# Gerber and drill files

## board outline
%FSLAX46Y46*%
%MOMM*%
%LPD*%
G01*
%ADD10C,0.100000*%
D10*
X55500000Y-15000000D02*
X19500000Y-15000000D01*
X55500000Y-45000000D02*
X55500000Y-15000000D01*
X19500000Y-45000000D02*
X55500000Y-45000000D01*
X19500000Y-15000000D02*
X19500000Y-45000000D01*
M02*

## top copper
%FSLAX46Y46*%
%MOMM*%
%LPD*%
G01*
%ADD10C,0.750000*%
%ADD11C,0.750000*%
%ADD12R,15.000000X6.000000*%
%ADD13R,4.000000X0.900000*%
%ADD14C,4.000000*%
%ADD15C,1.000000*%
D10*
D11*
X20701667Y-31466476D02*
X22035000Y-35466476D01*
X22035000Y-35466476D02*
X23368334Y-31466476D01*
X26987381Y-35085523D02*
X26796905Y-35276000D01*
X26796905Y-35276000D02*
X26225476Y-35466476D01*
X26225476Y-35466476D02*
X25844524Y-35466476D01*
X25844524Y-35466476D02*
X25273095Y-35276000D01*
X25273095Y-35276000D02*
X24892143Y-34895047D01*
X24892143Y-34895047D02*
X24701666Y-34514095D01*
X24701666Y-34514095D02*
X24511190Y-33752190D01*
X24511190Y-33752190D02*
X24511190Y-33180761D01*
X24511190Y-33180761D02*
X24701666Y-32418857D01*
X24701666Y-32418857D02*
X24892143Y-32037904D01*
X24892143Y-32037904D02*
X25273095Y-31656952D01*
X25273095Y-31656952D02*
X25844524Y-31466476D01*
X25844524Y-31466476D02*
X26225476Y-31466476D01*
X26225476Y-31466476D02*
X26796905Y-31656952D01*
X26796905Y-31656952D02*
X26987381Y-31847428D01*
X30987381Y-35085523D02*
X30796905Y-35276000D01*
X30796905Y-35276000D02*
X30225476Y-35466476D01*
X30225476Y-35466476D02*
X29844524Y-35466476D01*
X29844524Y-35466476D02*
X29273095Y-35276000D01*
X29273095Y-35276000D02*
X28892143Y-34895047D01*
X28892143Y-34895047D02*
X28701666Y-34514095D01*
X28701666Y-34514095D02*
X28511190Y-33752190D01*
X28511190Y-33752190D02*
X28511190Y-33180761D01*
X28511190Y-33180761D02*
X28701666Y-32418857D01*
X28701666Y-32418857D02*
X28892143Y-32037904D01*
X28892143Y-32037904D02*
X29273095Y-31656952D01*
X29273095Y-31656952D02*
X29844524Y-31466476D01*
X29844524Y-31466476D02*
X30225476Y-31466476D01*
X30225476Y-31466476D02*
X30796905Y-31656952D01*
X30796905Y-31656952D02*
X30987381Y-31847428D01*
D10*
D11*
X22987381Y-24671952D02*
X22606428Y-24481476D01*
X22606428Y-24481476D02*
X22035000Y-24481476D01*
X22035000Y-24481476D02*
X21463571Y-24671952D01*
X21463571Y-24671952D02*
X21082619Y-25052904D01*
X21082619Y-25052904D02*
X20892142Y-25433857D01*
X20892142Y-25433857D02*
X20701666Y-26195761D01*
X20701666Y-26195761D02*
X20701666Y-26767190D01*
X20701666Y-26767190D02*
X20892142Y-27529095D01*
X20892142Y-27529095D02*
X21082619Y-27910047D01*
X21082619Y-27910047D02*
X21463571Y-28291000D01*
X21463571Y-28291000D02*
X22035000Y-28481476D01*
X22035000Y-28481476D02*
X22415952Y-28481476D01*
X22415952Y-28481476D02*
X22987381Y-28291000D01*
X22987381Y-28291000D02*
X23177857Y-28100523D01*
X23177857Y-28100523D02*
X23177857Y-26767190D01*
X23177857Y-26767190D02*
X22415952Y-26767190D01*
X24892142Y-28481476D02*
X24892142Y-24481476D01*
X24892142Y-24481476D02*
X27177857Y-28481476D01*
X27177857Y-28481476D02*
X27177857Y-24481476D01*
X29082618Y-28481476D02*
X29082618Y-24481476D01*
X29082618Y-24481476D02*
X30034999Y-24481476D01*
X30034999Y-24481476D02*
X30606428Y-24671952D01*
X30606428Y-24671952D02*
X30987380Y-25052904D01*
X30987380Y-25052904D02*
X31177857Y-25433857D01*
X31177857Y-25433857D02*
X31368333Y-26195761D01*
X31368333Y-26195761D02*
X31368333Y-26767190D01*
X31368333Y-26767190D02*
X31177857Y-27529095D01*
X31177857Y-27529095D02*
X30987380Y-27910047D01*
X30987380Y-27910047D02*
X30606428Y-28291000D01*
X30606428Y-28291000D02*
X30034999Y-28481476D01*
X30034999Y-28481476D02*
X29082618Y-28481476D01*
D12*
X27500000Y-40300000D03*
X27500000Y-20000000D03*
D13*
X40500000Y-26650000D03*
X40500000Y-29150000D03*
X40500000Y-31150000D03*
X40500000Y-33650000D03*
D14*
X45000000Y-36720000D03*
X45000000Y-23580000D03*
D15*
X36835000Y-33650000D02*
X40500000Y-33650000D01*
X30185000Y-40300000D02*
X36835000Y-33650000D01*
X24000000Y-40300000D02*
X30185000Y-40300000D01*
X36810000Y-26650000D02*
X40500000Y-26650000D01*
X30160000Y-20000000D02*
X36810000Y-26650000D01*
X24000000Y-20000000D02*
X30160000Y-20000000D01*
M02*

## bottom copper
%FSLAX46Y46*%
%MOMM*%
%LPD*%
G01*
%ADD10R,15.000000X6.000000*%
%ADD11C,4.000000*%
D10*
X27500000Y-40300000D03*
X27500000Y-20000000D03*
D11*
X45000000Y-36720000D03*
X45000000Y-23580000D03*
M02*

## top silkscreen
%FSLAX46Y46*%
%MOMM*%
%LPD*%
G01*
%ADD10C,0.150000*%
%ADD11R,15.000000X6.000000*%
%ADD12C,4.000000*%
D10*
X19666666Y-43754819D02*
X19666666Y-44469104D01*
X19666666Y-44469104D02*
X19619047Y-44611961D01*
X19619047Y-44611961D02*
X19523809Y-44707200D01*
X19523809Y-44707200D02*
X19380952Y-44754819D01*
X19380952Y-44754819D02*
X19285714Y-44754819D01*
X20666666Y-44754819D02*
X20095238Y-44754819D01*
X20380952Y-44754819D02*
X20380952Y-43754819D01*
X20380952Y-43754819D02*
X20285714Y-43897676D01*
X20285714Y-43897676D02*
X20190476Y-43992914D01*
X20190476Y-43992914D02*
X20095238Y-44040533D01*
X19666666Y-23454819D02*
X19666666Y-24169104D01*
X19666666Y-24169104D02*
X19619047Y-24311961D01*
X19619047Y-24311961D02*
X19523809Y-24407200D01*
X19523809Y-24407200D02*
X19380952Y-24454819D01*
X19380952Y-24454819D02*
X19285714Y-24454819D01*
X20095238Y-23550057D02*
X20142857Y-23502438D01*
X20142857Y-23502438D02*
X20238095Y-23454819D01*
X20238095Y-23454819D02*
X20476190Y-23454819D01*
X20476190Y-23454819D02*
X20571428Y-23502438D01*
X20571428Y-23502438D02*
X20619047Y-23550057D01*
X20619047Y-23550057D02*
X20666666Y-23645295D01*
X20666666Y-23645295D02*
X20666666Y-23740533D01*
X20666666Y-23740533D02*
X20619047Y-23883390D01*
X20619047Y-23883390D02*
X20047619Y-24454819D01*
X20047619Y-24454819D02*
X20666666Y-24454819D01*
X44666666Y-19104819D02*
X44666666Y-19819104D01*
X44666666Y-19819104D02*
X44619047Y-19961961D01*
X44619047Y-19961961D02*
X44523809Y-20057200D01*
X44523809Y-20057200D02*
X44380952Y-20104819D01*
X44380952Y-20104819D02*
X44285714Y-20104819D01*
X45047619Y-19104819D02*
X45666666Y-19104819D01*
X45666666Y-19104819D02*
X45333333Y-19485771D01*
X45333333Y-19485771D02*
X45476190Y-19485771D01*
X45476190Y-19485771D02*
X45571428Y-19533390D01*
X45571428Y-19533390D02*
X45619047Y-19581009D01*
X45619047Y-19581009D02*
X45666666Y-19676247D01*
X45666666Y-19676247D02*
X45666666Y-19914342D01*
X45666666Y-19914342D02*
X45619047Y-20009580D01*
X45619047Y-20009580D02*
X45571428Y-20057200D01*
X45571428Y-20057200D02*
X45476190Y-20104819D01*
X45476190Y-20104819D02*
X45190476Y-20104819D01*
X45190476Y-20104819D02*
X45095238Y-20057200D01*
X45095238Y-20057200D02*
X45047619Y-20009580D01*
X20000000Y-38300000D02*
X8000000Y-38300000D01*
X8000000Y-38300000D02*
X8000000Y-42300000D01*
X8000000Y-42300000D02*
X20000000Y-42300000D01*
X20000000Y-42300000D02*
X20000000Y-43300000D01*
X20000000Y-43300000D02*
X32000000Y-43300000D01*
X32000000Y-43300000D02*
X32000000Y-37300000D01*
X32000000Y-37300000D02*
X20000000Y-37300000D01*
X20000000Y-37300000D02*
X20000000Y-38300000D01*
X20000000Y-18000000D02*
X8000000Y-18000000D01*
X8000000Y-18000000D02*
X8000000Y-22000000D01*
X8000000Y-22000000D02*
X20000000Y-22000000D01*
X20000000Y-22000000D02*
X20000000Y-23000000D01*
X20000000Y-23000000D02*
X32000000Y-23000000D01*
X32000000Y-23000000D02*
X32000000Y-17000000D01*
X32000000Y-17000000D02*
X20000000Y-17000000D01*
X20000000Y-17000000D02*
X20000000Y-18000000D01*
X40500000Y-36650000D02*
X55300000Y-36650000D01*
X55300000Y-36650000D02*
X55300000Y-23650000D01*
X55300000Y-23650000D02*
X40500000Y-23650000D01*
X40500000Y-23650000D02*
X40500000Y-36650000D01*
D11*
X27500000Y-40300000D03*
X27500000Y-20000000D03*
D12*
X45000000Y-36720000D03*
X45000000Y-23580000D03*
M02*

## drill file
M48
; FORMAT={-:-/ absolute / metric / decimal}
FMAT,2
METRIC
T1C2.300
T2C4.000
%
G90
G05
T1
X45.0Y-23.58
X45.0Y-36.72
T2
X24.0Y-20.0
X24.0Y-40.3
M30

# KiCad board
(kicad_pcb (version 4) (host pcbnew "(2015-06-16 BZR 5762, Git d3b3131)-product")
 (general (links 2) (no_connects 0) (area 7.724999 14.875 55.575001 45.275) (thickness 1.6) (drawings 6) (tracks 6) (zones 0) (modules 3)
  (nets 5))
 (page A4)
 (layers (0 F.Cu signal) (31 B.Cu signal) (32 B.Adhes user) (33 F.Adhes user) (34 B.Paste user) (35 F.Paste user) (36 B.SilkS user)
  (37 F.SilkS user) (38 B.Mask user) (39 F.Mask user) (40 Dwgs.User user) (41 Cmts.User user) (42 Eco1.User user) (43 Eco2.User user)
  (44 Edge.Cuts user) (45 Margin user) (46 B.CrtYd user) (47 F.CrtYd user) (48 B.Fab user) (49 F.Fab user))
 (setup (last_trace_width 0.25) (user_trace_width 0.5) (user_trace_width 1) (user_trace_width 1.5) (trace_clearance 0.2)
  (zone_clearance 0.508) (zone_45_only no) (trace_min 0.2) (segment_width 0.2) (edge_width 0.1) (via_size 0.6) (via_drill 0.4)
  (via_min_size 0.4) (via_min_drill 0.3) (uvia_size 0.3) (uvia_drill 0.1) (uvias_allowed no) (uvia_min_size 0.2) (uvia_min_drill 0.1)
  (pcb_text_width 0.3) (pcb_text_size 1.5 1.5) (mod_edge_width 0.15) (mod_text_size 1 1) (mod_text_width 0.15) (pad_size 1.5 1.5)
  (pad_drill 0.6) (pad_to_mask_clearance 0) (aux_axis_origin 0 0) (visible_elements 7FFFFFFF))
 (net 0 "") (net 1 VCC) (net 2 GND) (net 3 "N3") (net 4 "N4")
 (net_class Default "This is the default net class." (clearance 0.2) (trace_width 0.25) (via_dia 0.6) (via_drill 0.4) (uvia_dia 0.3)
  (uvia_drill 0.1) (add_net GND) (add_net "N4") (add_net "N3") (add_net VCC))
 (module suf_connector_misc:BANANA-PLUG (layer F.Cu) (at 20 40.3)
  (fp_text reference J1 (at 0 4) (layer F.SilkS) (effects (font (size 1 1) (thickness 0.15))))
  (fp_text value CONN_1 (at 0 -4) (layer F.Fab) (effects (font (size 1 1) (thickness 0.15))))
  (fp_line (start 0 -2) (end -12 -2) (layer F.SilkS) (width 0.15))
  (fp_line (start -12 -2) (end -12 2) (layer F.SilkS) (width 0.15))
  (fp_line (start -12 2) (end 0 2) (layer F.SilkS) (width 0.15)) (fp_line (start 0 2) (end 0 3) (layer F.SilkS) (width 0.15))
  (fp_line (start 0 3) (end 12 3) (layer F.SilkS) (width 0.15))
  (fp_line (start 12 3) (end 12 -3) (layer F.SilkS) (width 0.15))
  (fp_line (start 12 -3) (end 0 -3) (layer F.SilkS) (width 0.15))
  (fp_line (start 0 -3) (end 0 -2) (layer F.SilkS) (width 0.15))
  (pad 1 thru_hole rect (at 4 0) (size 15 6) (drill 4 (offset 3.5 0)) (layers *.Cu *.Mask F.SilkS) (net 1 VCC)))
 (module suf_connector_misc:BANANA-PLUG (layer F.Cu) (at 20 20)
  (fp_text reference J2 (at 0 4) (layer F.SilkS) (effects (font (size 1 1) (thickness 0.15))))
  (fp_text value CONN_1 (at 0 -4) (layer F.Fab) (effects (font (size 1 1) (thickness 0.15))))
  (fp_line (start 0 -2) (end -12 -2) (layer F.SilkS) (width 0.15))
  (fp_line (start -12 -2) (end -12 2) (layer F.SilkS) (width 0.15))
  (fp_line (start -12 2) (end 0 2) (layer F.SilkS) (width 0.15)) (fp_line (start 0 2) (end 0 3) (layer F.SilkS) (width 0.15))
  (fp_line (start 0 3) (end 12 3) (layer F.SilkS) (width 0.15))
  (fp_line (start 12 3) (end 12 -3) (layer F.SilkS) (width 0.15))
  (fp_line (start 12 -3) (end 0 -3) (layer F.SilkS) (width 0.15))
  (fp_line (start 0 -3) (end 0 -2) (layer F.SilkS) (width 0.15))
  (pad 1 thru_hole rect (at 4 0) (size 15 6) (drill 4 (offset 3.5 0)) (layers *.Cu *.Mask F.SilkS) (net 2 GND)))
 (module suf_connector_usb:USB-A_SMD (layer F.Cu) (at 45 30.15 180)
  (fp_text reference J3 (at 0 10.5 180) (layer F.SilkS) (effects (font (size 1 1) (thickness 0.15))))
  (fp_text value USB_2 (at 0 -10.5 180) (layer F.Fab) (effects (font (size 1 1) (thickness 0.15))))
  (fp_line (start 4.5 -6.5) (end -10.3 -6.5) (layer F.SilkS) (width 0.15))
  (fp_line (start -10.3 -6.5) (end -10.3 6.5) (layer F.SilkS) (width 0.15))
  (fp_line (start -10.3 6.5) (end 4.5 6.5) (layer F.SilkS) (width 0.15))
  (fp_line (start 4.5 6.5) (end 4.5 -6.5) (layer F.SilkS) (width 0.15))
  (pad 4 smd rect (at 4.5 3.5 180) (size 4 0.9) (layers F.Cu F.Paste F.Mask) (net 2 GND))
  (pad 3 smd rect (at 4.5 1 180) (size 4 0.9) (layers F.Cu F.Paste F.Mask) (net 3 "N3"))
  (pad 2 smd rect (at 4.5 -1 180) (size 4 0.9) (layers F.Cu F.Paste F.Mask) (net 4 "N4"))
  (pad 1 smd rect (at 4.5 -3.5 180) (size 4 0.9) (layers F.Cu F.Paste F.Mask) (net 1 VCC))
  (pad "" thru_hole circle (at 0 -6.57 180) (size 4 4) (drill 2.3) (layers *.Cu *.Mask F.SilkS))
  (pad "" thru_hole circle (at 0 6.57 180) (size 4 4) (drill 2.3) (layers *.Cu *.Mask F.SilkS)))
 (gr_line (start 55.5 15) (end 19.5 15) (angle 90) (layer Edge.Cuts) (width 0.1))
 (gr_line (start 55.5 45) (end 55.5 15) (angle 90) (layer Edge.Cuts) (width 0.1))
 (gr_line (start 19.5 45) (end 55.5 45) (angle 90) (layer Edge.Cuts) (width 0.1))
 (gr_line (start 19.5 15) (end 19.5 45) (angle 90) (layer Edge.Cuts) (width 0.1))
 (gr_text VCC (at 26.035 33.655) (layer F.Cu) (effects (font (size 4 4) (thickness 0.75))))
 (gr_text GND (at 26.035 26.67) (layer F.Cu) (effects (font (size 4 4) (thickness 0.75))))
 (segment (start 36.835 33.65) (end 40.5 33.65) (width 1) (layer F.Cu) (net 1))
 (segment (start 30.185 40.3) (end 36.835 33.65) (width 1) (layer F.Cu) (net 1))
 (segment (start 24 40.3) (end 30.185 40.3) (width 1) (layer F.Cu) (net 1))
 (segment (start 36.81 26.65) (end 40.5 26.65) (width 1) (layer F.Cu) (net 2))
 (segment (start 30.16 20) (end 36.81 26.65) (width 1) (layer F.Cu) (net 2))
 (segment (start 24 20) (end 30.16 20) (width 1) (layer F.Cu) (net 2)))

